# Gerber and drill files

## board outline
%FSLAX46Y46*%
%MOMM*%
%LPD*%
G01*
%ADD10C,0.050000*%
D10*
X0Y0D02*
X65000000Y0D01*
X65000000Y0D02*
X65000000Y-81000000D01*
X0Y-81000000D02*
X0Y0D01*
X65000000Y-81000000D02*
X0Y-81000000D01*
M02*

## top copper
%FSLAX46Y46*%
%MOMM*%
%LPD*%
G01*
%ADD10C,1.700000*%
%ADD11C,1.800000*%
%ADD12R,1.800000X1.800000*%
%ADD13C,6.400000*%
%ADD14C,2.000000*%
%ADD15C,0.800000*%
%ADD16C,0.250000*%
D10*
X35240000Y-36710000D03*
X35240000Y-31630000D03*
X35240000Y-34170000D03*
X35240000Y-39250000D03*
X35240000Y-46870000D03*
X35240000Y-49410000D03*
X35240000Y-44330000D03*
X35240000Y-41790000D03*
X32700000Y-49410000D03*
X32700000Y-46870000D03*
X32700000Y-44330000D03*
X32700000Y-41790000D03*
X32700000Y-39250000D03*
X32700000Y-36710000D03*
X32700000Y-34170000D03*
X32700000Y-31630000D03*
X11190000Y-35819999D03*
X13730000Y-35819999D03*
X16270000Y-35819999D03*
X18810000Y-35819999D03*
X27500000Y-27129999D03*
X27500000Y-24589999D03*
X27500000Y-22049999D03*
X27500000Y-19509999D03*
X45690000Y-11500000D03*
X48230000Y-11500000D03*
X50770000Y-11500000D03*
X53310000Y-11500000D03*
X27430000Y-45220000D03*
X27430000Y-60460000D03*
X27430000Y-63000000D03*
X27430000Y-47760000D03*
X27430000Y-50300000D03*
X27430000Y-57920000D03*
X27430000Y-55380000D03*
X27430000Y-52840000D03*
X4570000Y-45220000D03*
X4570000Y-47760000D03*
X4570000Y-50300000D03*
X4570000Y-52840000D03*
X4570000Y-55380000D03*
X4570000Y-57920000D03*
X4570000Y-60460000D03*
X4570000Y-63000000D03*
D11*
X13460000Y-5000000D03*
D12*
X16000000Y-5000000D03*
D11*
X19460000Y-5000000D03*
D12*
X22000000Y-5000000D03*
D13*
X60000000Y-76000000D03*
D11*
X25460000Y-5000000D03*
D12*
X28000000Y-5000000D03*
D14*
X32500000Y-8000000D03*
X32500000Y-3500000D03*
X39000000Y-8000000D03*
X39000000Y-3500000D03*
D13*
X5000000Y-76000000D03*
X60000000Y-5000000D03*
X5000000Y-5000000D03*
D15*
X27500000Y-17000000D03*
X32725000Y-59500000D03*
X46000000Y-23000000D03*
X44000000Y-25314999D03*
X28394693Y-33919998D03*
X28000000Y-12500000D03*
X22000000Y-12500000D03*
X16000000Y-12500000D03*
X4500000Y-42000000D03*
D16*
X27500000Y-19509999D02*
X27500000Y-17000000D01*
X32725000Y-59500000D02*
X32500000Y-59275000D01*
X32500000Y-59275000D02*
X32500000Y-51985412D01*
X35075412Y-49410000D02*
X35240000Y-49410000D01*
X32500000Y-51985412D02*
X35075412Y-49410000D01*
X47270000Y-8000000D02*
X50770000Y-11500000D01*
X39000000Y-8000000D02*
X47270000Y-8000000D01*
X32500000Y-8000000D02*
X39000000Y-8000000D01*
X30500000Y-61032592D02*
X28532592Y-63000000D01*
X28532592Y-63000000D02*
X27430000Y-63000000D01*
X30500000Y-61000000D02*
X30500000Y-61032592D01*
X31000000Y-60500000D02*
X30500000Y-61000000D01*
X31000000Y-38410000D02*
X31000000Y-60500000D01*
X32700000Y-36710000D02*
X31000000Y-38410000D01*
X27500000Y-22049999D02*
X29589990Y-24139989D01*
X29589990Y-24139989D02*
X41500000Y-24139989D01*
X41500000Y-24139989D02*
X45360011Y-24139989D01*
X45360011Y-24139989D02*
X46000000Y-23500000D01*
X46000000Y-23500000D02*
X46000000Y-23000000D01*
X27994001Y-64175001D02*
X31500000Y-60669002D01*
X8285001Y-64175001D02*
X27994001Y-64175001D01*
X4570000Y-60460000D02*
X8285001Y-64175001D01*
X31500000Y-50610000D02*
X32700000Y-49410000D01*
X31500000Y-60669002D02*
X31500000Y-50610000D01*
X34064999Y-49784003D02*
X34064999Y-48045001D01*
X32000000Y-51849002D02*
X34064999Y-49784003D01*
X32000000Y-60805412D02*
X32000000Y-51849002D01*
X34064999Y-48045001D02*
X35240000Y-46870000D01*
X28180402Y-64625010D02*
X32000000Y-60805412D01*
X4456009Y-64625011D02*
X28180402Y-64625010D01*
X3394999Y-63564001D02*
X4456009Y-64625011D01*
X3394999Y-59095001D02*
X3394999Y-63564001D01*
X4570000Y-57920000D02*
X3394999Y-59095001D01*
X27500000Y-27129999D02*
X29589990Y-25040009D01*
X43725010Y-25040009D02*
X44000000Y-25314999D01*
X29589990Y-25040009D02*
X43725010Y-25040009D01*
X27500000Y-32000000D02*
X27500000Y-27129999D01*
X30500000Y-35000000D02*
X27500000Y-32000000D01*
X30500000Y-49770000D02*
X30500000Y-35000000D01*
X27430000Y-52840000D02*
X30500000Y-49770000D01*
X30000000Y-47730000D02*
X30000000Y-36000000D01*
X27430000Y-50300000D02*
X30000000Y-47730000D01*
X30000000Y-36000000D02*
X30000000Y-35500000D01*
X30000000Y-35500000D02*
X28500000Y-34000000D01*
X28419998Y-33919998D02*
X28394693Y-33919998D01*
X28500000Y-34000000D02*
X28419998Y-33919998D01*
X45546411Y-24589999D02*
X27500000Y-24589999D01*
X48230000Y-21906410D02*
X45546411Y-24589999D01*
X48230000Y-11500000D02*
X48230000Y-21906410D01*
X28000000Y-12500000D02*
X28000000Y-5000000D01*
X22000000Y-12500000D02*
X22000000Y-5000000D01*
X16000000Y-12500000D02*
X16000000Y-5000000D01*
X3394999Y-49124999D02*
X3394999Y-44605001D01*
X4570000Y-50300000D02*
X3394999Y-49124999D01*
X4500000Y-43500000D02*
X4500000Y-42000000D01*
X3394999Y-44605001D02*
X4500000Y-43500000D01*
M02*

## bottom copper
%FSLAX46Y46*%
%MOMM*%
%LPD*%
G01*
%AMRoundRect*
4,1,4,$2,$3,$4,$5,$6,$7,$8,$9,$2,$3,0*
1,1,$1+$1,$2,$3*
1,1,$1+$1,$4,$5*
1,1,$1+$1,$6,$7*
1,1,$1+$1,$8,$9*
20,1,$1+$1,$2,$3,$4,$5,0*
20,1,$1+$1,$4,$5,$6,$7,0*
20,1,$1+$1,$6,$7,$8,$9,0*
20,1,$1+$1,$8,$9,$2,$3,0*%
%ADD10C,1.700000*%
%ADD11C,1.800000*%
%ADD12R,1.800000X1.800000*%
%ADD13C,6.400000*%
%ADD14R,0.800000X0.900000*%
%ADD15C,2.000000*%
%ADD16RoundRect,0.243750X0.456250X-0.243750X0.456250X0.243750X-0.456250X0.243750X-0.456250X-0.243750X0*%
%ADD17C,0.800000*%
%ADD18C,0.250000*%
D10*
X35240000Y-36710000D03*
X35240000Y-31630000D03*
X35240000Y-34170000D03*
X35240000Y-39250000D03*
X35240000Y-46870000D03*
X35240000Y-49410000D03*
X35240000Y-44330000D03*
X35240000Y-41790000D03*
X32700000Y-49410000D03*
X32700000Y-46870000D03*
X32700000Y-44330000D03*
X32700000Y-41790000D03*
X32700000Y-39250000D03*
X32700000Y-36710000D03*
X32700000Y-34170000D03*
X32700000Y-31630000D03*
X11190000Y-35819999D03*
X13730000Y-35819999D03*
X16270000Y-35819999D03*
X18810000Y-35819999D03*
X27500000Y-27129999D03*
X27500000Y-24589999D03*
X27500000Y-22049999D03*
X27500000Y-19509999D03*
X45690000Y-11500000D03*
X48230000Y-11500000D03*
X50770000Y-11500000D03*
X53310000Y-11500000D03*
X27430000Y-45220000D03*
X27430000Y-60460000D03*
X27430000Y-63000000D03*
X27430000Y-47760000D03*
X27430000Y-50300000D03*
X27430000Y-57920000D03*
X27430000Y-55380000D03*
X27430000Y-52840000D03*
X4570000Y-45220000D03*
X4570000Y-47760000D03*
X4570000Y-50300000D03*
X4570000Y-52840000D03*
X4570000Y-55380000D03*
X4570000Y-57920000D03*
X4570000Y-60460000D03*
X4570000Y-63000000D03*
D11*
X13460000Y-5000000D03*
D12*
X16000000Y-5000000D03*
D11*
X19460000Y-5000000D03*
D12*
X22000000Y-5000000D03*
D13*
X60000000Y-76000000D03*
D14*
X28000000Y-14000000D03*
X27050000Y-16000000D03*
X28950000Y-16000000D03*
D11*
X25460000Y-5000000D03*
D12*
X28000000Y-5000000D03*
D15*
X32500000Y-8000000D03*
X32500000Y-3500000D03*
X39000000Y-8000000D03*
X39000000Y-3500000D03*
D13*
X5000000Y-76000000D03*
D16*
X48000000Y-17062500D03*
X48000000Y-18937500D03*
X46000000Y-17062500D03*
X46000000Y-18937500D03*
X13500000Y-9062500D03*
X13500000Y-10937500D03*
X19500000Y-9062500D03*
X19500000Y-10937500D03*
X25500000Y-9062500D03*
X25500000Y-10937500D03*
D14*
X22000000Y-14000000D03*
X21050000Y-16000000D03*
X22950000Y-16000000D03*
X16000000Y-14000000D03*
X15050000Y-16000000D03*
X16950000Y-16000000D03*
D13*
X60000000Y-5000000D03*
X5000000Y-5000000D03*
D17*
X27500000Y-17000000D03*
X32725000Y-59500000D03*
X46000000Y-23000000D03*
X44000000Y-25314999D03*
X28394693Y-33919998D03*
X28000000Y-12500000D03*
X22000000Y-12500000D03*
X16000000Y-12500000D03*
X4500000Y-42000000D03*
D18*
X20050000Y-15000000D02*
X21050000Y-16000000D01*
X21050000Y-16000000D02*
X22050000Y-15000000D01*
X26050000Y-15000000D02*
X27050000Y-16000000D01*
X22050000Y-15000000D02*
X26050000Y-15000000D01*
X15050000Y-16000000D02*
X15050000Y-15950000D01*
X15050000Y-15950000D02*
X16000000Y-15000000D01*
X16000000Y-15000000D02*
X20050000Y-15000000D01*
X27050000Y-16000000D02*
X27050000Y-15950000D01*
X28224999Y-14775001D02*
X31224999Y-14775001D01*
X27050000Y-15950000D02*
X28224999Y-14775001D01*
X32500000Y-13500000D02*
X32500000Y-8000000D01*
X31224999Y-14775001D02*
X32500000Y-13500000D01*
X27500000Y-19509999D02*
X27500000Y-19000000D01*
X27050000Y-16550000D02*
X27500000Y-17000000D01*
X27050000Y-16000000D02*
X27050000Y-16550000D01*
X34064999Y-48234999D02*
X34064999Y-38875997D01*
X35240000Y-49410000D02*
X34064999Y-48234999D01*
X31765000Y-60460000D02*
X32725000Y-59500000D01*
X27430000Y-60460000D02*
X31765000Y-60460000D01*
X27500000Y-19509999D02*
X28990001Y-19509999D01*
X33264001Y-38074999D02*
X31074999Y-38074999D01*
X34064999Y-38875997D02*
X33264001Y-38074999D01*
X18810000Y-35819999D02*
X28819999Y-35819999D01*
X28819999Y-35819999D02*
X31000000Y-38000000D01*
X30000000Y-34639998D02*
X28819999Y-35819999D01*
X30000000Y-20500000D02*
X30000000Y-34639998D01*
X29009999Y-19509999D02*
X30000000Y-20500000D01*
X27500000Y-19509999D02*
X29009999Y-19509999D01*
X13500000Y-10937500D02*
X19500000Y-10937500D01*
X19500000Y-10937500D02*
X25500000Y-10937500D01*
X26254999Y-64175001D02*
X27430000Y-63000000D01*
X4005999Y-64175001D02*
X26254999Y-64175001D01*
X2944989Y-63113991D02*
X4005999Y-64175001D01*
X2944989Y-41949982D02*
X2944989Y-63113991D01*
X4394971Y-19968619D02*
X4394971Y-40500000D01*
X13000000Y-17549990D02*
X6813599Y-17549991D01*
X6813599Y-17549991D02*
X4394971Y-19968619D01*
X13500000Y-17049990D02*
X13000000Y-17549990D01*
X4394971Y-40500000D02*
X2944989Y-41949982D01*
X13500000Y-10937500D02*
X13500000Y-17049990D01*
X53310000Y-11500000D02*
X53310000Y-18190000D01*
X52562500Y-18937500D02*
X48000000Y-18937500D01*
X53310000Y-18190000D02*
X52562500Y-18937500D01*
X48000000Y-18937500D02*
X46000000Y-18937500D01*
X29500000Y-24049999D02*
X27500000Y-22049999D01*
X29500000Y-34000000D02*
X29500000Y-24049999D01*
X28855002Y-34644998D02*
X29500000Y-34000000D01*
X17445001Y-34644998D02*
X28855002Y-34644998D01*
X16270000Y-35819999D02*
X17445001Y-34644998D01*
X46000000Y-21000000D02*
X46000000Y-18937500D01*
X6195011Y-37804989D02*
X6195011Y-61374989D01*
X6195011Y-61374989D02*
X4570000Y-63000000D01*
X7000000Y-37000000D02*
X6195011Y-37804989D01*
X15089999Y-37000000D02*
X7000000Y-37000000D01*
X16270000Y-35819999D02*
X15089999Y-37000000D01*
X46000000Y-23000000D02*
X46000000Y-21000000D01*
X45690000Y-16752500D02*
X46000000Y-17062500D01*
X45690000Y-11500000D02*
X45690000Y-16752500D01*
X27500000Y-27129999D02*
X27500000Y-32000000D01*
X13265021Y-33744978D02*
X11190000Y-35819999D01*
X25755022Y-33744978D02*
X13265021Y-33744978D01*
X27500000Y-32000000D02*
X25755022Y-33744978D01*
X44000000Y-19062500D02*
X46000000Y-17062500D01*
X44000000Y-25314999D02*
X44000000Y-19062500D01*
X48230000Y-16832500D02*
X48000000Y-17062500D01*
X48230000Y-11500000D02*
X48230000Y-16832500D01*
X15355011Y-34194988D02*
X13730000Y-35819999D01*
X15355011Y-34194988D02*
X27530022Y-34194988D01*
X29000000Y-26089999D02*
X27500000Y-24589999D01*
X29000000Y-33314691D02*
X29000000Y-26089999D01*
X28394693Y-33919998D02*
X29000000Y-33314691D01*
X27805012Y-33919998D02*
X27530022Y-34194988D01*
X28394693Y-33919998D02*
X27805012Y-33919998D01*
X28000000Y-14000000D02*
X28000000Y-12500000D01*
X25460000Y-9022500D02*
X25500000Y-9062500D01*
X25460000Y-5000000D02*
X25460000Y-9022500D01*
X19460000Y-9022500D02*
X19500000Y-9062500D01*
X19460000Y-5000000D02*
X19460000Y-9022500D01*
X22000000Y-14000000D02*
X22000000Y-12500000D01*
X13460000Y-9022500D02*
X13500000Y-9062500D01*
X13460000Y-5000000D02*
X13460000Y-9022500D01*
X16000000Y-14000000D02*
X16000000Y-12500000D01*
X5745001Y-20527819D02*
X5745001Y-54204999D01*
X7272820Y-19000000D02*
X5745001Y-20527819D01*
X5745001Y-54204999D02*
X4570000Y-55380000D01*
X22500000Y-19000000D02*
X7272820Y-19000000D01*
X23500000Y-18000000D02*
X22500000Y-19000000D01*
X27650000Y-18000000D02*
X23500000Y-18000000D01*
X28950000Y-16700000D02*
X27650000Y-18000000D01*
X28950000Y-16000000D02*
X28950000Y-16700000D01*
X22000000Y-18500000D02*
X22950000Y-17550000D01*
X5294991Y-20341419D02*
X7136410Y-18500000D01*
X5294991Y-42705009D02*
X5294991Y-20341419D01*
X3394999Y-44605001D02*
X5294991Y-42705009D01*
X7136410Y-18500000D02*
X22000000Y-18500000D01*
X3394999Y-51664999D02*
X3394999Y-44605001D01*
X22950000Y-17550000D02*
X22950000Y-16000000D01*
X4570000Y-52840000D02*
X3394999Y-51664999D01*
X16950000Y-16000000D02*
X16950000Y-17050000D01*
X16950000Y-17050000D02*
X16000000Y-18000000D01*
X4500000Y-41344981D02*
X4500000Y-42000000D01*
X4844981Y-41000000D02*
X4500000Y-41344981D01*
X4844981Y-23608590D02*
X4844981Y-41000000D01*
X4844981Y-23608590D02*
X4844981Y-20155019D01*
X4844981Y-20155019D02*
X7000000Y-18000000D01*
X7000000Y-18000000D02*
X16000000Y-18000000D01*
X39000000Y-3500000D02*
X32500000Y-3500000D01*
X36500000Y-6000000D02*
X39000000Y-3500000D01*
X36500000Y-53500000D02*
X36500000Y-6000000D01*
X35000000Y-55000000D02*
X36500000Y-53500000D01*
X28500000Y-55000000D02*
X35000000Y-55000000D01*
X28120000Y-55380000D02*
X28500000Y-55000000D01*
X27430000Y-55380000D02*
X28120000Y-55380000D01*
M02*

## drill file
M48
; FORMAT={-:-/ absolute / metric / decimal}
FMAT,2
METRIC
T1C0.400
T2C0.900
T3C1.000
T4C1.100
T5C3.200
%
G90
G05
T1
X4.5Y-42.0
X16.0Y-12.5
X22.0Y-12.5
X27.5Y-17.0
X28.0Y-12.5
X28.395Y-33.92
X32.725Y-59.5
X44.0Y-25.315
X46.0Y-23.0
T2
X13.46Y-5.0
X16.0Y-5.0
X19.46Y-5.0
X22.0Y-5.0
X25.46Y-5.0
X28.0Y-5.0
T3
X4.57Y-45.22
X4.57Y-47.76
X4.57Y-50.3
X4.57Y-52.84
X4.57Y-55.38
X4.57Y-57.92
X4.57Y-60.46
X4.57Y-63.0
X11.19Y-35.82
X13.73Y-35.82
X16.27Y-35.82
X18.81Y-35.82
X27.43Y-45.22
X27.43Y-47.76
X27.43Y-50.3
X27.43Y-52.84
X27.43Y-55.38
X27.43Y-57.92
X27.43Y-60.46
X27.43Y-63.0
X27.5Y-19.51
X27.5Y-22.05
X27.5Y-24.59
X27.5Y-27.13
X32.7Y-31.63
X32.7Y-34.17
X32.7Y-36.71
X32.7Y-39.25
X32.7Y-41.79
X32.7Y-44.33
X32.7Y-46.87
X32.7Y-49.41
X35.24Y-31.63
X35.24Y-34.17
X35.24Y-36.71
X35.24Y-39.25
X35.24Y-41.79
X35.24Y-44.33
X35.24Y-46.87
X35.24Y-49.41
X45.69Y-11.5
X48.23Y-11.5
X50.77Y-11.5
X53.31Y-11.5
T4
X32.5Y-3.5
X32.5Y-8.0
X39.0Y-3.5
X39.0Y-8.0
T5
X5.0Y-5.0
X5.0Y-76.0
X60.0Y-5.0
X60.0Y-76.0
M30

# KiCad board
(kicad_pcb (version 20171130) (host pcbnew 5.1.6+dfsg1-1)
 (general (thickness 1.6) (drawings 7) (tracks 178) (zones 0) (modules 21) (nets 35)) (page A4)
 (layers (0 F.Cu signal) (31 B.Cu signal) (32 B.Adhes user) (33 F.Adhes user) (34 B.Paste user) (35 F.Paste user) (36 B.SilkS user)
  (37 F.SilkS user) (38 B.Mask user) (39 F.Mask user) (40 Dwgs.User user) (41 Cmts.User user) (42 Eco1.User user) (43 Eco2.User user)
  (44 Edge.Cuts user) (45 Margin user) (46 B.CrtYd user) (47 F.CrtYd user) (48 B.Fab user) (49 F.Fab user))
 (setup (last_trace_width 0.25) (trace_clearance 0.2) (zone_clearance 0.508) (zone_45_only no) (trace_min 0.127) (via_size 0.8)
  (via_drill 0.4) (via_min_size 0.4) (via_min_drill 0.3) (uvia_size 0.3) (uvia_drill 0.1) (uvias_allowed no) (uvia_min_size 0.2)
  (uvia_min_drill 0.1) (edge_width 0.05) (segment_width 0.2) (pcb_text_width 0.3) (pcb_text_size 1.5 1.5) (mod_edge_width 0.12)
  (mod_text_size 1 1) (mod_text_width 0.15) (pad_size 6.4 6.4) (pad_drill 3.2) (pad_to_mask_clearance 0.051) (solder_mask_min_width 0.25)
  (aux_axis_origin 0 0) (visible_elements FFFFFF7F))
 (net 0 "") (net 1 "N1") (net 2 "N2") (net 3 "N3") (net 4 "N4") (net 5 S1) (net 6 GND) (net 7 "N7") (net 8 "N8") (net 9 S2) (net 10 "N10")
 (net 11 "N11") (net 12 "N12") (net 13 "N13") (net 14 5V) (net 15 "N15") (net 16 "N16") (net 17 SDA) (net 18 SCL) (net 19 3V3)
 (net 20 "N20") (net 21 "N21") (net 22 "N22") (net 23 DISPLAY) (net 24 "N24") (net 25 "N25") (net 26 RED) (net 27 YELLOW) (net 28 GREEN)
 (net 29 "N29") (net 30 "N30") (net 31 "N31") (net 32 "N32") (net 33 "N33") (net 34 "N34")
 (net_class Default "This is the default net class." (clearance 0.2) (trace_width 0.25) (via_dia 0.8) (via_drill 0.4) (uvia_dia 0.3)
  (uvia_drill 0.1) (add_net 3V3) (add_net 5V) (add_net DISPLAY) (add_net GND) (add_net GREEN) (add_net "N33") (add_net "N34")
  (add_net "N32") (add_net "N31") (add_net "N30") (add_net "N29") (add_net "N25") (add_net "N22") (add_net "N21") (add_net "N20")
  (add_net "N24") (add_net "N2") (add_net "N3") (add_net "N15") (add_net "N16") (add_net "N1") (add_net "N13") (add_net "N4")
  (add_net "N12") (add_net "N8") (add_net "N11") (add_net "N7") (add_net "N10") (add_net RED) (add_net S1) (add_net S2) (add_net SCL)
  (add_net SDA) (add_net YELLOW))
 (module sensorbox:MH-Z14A (layer F.Cu) (at 65 14.5 270)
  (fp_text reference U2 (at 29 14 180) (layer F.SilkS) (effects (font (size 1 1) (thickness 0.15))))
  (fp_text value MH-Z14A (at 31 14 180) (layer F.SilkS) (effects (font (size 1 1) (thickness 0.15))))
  (pad 2 thru_hole circle (at 22.21 29.76 270) (size 1.7 1.7) (drill 1) (layers *.Cu *.Mask) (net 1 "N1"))
  (pad 14 thru_hole circle (at 17.13 29.76 270) (size 1.7 1.7) (drill 1) (layers *.Cu *.Mask) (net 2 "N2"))
  (pad 15 thru_hole circle (at 19.67 29.76 270) (size 1.7 1.7) (drill 1) (layers *.Cu *.Mask) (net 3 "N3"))
  (pad 4 thru_hole circle (at 24.75 29.76 270) (size 1.7 1.7) (drill 1) (layers *.Cu *.Mask) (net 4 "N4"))
  (pad 10 thru_hole circle (at 32.37 29.76 270) (size 1.7 1.7) (drill 1) (layers *.Cu *.Mask) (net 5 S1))
  (pad 12 thru_hole circle (at 34.91 29.76 270) (size 1.7 1.7) (drill 1) (layers *.Cu *.Mask) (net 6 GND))
  (pad 8 thru_hole circle (at 29.83 29.76 270) (size 1.7 1.7) (drill 1) (layers *.Cu *.Mask) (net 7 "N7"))
  (pad 6 thru_hole circle (at 27.29 29.76 270) (size 1.7 1.7) (drill 1) (layers *.Cu *.Mask) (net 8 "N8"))
  (pad 11 thru_hole circle (at 34.91 32.3 270) (size 1.7 1.7) (drill 1) (layers *.Cu *.Mask) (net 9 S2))
  (pad 9 thru_hole circle (at 32.37 32.3 270) (size 1.7 1.7) (drill 1) (layers *.Cu *.Mask) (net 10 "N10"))
  (pad 7 thru_hole circle (at 29.83 32.3 270) (size 1.7 1.7) (drill 1) (layers *.Cu *.Mask) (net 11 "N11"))
  (pad 5 thru_hole circle (at 27.29 32.3 270) (size 1.7 1.7) (drill 1) (layers *.Cu *.Mask) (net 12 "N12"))
  (pad 3 thru_hole circle (at 24.75 32.3 270) (size 1.7 1.7) (drill 1) (layers *.Cu *.Mask) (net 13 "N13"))
  (pad 1 thru_hole circle (at 22.21 32.3 270) (size 1.7 1.7) (drill 1) (layers *.Cu *.Mask) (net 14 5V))
  (pad 16 thru_hole circle (at 19.67 32.3 270) (size 1.7 1.7) (drill 1) (layers *.Cu *.Mask) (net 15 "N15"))
  (pad 17 thru_hole circle (at 17.13 32.3 270) (size 1.7 1.7) (drill 1) (layers *.Cu *.Mask) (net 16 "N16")))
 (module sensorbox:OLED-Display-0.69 (layer F.Cu) (at 15 23.319999 180)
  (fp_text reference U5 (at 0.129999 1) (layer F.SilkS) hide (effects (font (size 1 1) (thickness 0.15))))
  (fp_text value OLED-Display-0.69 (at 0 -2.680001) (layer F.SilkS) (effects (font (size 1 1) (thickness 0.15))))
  (pad 4 thru_hole circle (at 3.81 -12.5 180) (size 1.7 1.7) (drill 1) (layers *.Cu *.Mask) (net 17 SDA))
  (pad 3 thru_hole circle (at 1.27 -12.5 180) (size 1.7 1.7) (drill 1) (layers *.Cu *.Mask) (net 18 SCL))
  (pad 2 thru_hole circle (at -1.27 -12.5 180) (size 1.7 1.7) (drill 1) (layers *.Cu *.Mask) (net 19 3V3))
  (pad 1 thru_hole circle (at -3.81 -12.5 180) (size 1.7 1.7) (drill 1) (layers *.Cu *.Mask) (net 6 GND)))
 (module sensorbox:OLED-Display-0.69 (layer F.Cu) (at 15 23.319999 270)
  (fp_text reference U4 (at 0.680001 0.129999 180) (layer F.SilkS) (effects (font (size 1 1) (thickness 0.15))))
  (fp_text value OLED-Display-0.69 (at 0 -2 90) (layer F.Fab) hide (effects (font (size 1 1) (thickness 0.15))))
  (pad 4 thru_hole circle (at 3.81 -12.5 270) (size 1.7 1.7) (drill 1) (layers *.Cu *.Mask) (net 17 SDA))
  (pad 3 thru_hole circle (at 1.27 -12.5 270) (size 1.7 1.7) (drill 1) (layers *.Cu *.Mask) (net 18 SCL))
  (pad 2 thru_hole circle (at -1.27 -12.5 270) (size 1.7 1.7) (drill 1) (layers *.Cu *.Mask) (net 19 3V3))
  (pad 1 thru_hole circle (at -3.81 -12.5 270) (size 1.7 1.7) (drill 1) (layers *.Cu *.Mask) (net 6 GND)))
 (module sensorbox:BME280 (layer F.Cu) (at 49.5 7 180)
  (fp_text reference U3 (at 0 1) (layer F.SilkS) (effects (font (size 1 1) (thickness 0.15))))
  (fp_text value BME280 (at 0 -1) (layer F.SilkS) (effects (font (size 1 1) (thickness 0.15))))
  (pad 4 thru_hole circle (at 3.81 -4.5 180) (size 1.7 1.7) (drill 1) (layers *.Cu *.Mask) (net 17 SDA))
  (pad 3 thru_hole circle (at 1.27 -4.5 180) (size 1.7 1.7) (drill 1) (layers *.Cu *.Mask) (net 18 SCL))
  (pad 2 thru_hole circle (at -1.27 -4.5 180) (size 1.7 1.7) (drill 1) (layers *.Cu *.Mask) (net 6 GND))
  (pad 1 thru_hole circle (at -3.81 -4.5 180) (size 1.7 1.7) (drill 1) (layers *.Cu *.Mask) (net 19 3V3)))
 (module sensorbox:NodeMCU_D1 (layer F.Cu) (at 16 72 90)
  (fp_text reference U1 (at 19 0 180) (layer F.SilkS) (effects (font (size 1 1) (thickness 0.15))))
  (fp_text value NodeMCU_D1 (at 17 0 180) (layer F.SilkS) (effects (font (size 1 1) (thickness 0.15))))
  (pad 8 thru_hole circle (at 26.78 11.43 90) (size 1.7 1.7) (drill 1) (layers *.Cu *.Mask) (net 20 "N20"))
  (pad 2 thru_hole circle (at 11.54 11.43 90) (size 1.7 1.7) (drill 1) (layers *.Cu *.Mask) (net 6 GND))
  (pad 1 thru_hole circle (at 9 11.43 90) (size 1.7 1.7) (drill 1) (layers *.Cu *.Mask) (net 14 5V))
  (pad 7 thru_hole circle (at 24.24 11.43 90) (size 1.7 1.7) (drill 1) (layers *.Cu *.Mask) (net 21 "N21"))
  (pad 6 thru_hole circle (at 21.7 11.43 90) (size 1.7 1.7) (drill 1) (layers *.Cu *.Mask) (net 18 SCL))
  (pad 3 thru_hole circle (at 14.08 11.43 90) (size 1.7 1.7) (drill 1) (layers *.Cu *.Mask) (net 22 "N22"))
  (pad 4 thru_hole circle (at 16.62 11.43 90) (size 1.7 1.7) (drill 1) (layers *.Cu *.Mask) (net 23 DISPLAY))
  (pad 5 thru_hole circle (at 19.16 11.43 90) (size 1.7 1.7) (drill 1) (layers *.Cu *.Mask) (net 17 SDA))
  (pad 9 thru_hole circle (at 26.78 -11.43 90) (size 1.7 1.7) (drill 1) (layers *.Cu *.Mask) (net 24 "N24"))
  (pad 10 thru_hole circle (at 24.24 -11.43 90) (size 1.7 1.7) (drill 1) (layers *.Cu *.Mask) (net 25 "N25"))
  (pad 11 thru_hole circle (at 21.7 -11.43 90) (size 1.7 1.7) (drill 1) (layers *.Cu *.Mask) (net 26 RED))
  (pad 12 thru_hole circle (at 19.16 -11.43 90) (size 1.7 1.7) (drill 1) (layers *.Cu *.Mask) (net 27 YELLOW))
  (pad 13 thru_hole circle (at 16.62 -11.43 90) (size 1.7 1.7) (drill 1) (layers *.Cu *.Mask) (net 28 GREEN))
  (pad 14 thru_hole circle (at 14.08 -11.43 90) (size 1.7 1.7) (drill 1) (layers *.Cu *.Mask) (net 5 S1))
  (pad 15 thru_hole circle (at 11.54 -11.43 90) (size 1.7 1.7) (drill 1) (layers *.Cu *.Mask) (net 9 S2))
  (pad 16 thru_hole circle (at 9 -11.43 90) (size 1.7 1.7) (drill 1) (layers *.Cu *.Mask) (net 19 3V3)))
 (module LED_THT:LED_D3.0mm (layer F.Cu) (at 16 5 180)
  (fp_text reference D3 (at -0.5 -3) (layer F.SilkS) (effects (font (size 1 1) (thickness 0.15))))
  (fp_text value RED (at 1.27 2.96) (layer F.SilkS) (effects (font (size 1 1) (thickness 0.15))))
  (pad 2 thru_hole circle (at 2.54 0 180) (size 1.8 1.8) (drill 0.9) (layers *.Cu *.Mask) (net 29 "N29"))
  (pad 1 thru_hole rect (at 0 0 180) (size 1.8 1.8) (drill 0.9) (layers *.Cu *.Mask) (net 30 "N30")))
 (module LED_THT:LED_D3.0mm (layer F.Cu) (at 22 5 180)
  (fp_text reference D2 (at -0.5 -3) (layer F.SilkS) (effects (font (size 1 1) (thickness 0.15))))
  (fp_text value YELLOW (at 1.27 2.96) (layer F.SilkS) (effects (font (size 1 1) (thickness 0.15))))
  (pad 2 thru_hole circle (at 2.54 0 180) (size 1.8 1.8) (drill 0.9) (layers *.Cu *.Mask) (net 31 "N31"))
  (pad 1 thru_hole rect (at 0 0 180) (size 1.8 1.8) (drill 0.9) (layers *.Cu *.Mask) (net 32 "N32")))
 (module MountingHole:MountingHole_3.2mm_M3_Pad (layer F.Cu) (at 60 76)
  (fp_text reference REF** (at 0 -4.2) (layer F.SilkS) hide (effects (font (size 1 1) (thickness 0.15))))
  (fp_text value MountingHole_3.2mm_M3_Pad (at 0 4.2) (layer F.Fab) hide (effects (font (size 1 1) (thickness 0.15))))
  (pad 1 thru_hole circle (at 0 0) (size 6.4 6.4) (drill 3.2) (layers *.Cu *.Mask)))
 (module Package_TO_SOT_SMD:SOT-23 (layer B.Cu) (at 28 15 90)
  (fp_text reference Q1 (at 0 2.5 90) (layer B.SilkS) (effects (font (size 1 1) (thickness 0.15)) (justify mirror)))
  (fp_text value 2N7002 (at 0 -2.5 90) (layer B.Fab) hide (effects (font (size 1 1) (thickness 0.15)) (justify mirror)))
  (pad 3 smd rect (at 1 0 90) (size 0.9 0.8) (layers B.Cu B.Paste B.Mask) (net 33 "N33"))
  (pad 2 smd rect (at -1 -0.95 90) (size 0.9 0.8) (layers B.Cu B.Paste B.Mask) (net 6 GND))
  (pad 1 smd rect (at -1 0.95 90) (size 0.9 0.8) (layers B.Cu B.Paste B.Mask) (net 28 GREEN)))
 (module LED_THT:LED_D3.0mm (layer F.Cu) (at 28 5 180)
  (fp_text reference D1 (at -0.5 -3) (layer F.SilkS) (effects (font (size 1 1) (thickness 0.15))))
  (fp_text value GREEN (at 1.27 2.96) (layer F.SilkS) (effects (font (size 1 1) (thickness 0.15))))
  (pad 2 thru_hole circle (at 2.54 0 180) (size 1.8 1.8) (drill 0.9) (layers *.Cu *.Mask) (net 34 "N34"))
  (pad 1 thru_hole rect (at 0 0 180) (size 1.8 1.8) (drill 0.9) (layers *.Cu *.Mask) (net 33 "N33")))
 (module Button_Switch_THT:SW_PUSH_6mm (layer F.Cu) (at 39 8 180)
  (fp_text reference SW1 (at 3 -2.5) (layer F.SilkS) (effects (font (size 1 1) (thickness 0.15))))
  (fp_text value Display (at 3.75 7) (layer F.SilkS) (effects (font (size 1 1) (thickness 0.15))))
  (pad 1 thru_hole circle (at 6.5 0 270) (size 2 2) (drill 1.1) (layers *.Cu *.Mask) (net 6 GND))
  (pad 2 thru_hole circle (at 6.5 4.5 270) (size 2 2) (drill 1.1) (layers *.Cu *.Mask) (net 23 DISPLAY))
  (pad 1 thru_hole circle (at 0 0 270) (size 2 2) (drill 1.1) (layers *.Cu *.Mask) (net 6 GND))
  (pad 2 thru_hole circle (at 0 4.5 270) (size 2 2) (drill 1.1) (layers *.Cu *.Mask) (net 23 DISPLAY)))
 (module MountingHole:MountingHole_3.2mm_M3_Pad (layer F.Cu) (at 5 76)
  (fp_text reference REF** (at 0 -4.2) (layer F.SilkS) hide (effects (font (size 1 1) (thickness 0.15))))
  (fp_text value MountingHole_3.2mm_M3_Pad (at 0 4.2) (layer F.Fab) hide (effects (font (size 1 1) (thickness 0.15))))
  (pad 1 thru_hole circle (at 0 0) (size 6.4 6.4) (drill 3.2) (layers *.Cu *.Mask)))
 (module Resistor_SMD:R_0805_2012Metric (layer B.Cu) (at 48 18 90)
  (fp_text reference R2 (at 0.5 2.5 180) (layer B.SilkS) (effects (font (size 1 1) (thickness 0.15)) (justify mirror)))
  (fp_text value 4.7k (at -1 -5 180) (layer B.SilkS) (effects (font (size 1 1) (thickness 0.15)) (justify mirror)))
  (pad 2 smd roundrect (at 0.9375 0 90) (size 0.975 1.4) (layers B.Cu B.Paste B.Mask) (roundrect_rratio 0.25) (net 18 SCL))
  (pad 1 smd roundrect (at -0.9375 0 90) (size 0.975 1.4) (layers B.Cu B.Paste B.Mask) (roundrect_rratio 0.25) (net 19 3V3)))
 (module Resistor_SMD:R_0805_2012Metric (layer B.Cu) (at 46 18 90)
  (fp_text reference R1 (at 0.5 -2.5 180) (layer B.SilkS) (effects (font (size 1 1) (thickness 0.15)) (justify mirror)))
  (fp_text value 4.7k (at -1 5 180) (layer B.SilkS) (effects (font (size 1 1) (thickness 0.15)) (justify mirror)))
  (pad 2 smd roundrect (at 0.9375 0 90) (size 0.975 1.4) (layers B.Cu B.Paste B.Mask) (roundrect_rratio 0.25) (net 17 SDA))
  (pad 1 smd roundrect (at -0.9375 0 90) (size 0.975 1.4) (layers B.Cu B.Paste B.Mask) (roundrect_rratio 0.25) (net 19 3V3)))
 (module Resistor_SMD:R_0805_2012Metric (layer B.Cu) (at 13.5 10 90)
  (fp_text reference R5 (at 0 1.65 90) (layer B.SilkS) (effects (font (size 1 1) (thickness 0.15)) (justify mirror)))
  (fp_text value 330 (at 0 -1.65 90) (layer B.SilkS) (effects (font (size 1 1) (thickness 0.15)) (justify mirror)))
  (pad 2 smd roundrect (at 0.9375 0 90) (size 0.975 1.4) (layers B.Cu B.Paste B.Mask) (roundrect_rratio 0.25) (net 29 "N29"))
  (pad 1 smd roundrect (at -0.9375 0 90) (size 0.975 1.4) (layers B.Cu B.Paste B.Mask) (roundrect_rratio 0.25) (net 14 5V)))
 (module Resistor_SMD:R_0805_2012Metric (layer B.Cu) (at 19.5 10 90)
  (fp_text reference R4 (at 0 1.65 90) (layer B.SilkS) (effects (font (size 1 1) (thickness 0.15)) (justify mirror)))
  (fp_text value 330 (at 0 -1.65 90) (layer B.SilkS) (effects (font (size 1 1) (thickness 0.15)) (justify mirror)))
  (pad 2 smd roundrect (at 0.9375 0 90) (size 0.975 1.4) (layers B.Cu B.Paste B.Mask) (roundrect_rratio 0.25) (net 31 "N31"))
  (pad 1 smd roundrect (at -0.9375 0 90) (size 0.975 1.4) (layers B.Cu B.Paste B.Mask) (roundrect_rratio 0.25) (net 14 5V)))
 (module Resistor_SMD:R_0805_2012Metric (layer B.Cu) (at 25.5 10 90)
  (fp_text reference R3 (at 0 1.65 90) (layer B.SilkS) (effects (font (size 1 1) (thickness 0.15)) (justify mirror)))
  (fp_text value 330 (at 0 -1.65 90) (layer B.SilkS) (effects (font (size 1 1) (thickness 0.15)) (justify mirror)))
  (pad 2 smd roundrect (at 0.9375 0 90) (size 0.975 1.4) (layers B.Cu B.Paste B.Mask) (roundrect_rratio 0.25) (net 34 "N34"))
  (pad 1 smd roundrect (at -0.9375 0 90) (size 0.975 1.4) (layers B.Cu B.Paste B.Mask) (roundrect_rratio 0.25) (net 14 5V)))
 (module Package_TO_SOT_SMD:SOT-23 (layer B.Cu) (at 22 15 90)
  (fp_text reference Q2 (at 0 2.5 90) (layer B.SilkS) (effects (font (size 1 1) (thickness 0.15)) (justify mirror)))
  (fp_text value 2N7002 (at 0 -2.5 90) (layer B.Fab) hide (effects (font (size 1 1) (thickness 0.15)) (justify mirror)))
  (pad 3 smd rect (at 1 0 90) (size 0.9 0.8) (layers B.Cu B.Paste B.Mask) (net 32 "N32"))
  (pad 2 smd rect (at -1 -0.95 90) (size 0.9 0.8) (layers B.Cu B.Paste B.Mask) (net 6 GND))
  (pad 1 smd rect (at -1 0.95 90) (size 0.9 0.8) (layers B.Cu B.Paste B.Mask) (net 27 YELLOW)))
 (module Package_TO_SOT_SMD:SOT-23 (layer B.Cu) (at 16 15 90)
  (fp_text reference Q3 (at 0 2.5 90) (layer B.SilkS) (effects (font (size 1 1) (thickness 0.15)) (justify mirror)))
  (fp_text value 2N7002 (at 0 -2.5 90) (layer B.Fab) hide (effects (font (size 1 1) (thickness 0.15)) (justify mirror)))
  (pad 3 smd rect (at 1 0 90) (size 0.9 0.8) (layers B.Cu B.Paste B.Mask) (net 30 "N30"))
  (pad 2 smd rect (at -1 -0.95 90) (size 0.9 0.8) (layers B.Cu B.Paste B.Mask) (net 6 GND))
  (pad 1 smd rect (at -1 0.95 90) (size 0.9 0.8) (layers B.Cu B.Paste B.Mask) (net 26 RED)))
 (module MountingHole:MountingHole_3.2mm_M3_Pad (layer F.Cu) (at 60 5)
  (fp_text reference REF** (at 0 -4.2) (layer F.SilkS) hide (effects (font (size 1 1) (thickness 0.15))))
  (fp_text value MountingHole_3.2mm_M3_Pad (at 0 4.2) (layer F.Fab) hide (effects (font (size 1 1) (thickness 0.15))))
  (pad 1 thru_hole circle (at 0 0) (size 6.4 6.4) (drill 3.2) (layers *.Cu *.Mask)))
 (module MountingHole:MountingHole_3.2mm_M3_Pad (layer F.Cu) (at 5 5)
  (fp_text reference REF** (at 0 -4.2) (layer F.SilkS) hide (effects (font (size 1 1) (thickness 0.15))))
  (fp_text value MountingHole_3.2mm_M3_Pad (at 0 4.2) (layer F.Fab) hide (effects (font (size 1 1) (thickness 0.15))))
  (pad 1 thru_hole circle (at 0 0) (size 6.4 6.4) (drill 3.2) (layers *.Cu *.Mask)))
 (gr_line (start 0 0) (end 65 0) (layer Edge.Cuts) (width 0.05))
 (gr_line (start 65 0) (end 65 81) (layer Edge.Cuts) (width 0.05))
 (gr_line (start 0 81) (end 0 0) (layer Edge.Cuts) (width 0.05))
 (gr_line (start 65 81) (end 0 81) (layer Edge.Cuts) (width 0.05))
 (segment (start 20.05 15) (end 21.05 16) (width 0.25) (layer B.Cu) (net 6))
 (segment (start 21.05 16) (end 22.05 15) (width 0.25) (layer B.Cu) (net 6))
 (segment (start 26.05 15) (end 27.05 16) (width 0.25) (layer B.Cu) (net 6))
 (segment (start 22.05 15) (end 26.05 15) (width 0.25) (layer B.Cu) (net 6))
 (segment (start 15.05 16) (end 15.05 15.95) (width 0.25) (layer B.Cu) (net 6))
 (segment (start 15.05 15.95) (end 16 15) (width 0.25) (layer B.Cu) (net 6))
 (segment (start 16 15) (end 20.05 15) (width 0.25) (layer B.Cu) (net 6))
 (segment (start 27.05 16) (end 27.05 15.95) (width 0.25) (layer B.Cu) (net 6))
 (segment (start 28.224999 14.775001) (end 31.224999 14.775001) (width 0.25) (layer B.Cu) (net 6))
 (segment (start 27.05 15.95) (end 28.224999 14.775001) (width 0.25) (layer B.Cu) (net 6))
 (segment (start 32.5 13.5) (end 32.5 8) (width 0.25) (layer B.Cu) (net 6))
 (segment (start 31.224999 14.775001) (end 32.5 13.5) (width 0.25) (layer B.Cu) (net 6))
 (segment (start 27.5 19.509999) (end 27.5 19) (width 0.25) (layer B.Cu) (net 6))
 (via (at 27.5 17) (size 0.8) (drill 0.4) (layers F.Cu B.Cu) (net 6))
 (segment (start 27.5 19.509999) (end 27.5 17) (width 0.25) (layer F.Cu) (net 6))
 (segment (start 27.05 16.55) (end 27.5 17) (width 0.25) (layer B.Cu) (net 6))
 (segment (start 27.05 16) (end 27.05 16.55) (width 0.25) (layer B.Cu) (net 6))
 (segment (start 34.064999 48.234999) (end 34.064999 38.875997) (width 0.25) (layer B.Cu) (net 6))
 (segment (start 35.24 49.41) (end 34.064999 48.234999) (width 0.25) (layer B.Cu) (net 6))
 (via (at 32.725 59.5) (size 0.8) (drill 0.4) (layers F.Cu B.Cu) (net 6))
 (segment (start 31.765 60.46) (end 32.725 59.5) (width 0.25) (layer B.Cu) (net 6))
 (segment (start 27.43 60.46) (end 31.765 60.46) (width 0.25) (layer B.Cu) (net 6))
 (segment (start 32.725 59.5) (end 32.5 59.275) (width 0.25) (layer F.Cu) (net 6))
 (segment (start 32.5 59.275) (end 32.5 51.985412) (width 0.25) (layer F.Cu) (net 6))
 (segment (start 35.075412 49.41) (end 35.24 49.41) (width 0.25) (layer F.Cu) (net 6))
 (segment (start 32.5 51.985412) (end 35.075412 49.41) (width 0.25) (layer F.Cu) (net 6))
 (segment (start 47.27 8) (end 50.77 11.5) (width 0.25) (layer F.Cu) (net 6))
 (segment (start 39 8) (end 47.27 8) (width 0.25) (layer F.Cu) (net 6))
 (segment (start 32.5 8) (end 39 8) (width 0.25) (layer F.Cu) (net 6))
 (segment (start 27.5 19.509999) (end 28.990001 19.509999) (width 0.25) (layer B.Cu) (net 6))
 (segment (start 33.264001 38.074999) (end 31.074999 38.074999) (width 0.25) (layer B.Cu) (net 6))
 (segment (start 34.064999 38.875997) (end 33.264001 38.074999) (width 0.25) (layer B.Cu) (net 6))
 (segment (start 18.81 35.819999) (end 28.819999 35.819999) (width 0.25) (layer B.Cu) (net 6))
 (segment (start 28.819999 35.819999) (end 31 38) (width 0.25) (layer B.Cu) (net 6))
 (segment (start 30 34.639998) (end 28.819999 35.819999) (width 0.25) (layer B.Cu) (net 6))
 (segment (start 30 20.5) (end 30 34.639998) (width 0.25) (layer B.Cu) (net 6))
 (segment (start 29.009999 19.509999) (end 30 20.5) (width 0.25) (layer B.Cu) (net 6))
 (segment (start 27.5 19.509999) (end 29.009999 19.509999) (width 0.25) (layer B.Cu) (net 6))
 (segment (start 13.5 10.9375) (end 19.5 10.9375) (width 0.25) (layer B.Cu) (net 14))
 (segment (start 19.5 10.9375) (end 25.5 10.9375) (width 0.25) (layer B.Cu) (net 14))
 (segment (start 26.254999 64.175001) (end 27.43 63) (width 0.25) (layer B.Cu) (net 14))
 (segment (start 4.005999 64.175001) (end 26.254999 64.175001) (width 0.25) (layer B.Cu) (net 14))
 (segment (start 2.944989 63.113991) (end 4.005999 64.175001) (width 0.25) (layer B.Cu) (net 14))
 (segment (start 2.944989 41.949982) (end 2.944989 63.113991) (width 0.25) (layer B.Cu) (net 14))
 (segment (start 4.394971 19.968619) (end 4.394971 40.5) (width 0.25) (layer B.Cu) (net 14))
 (segment (start 13 17.54999) (end 6.813599 17.549991) (width 0.25) (layer B.Cu) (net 14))
 (segment (start 6.813599 17.549991) (end 4.394971 19.968619) (width 0.25) (layer B.Cu) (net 14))
 (segment (start 13.5 17.04999) (end 13 17.54999) (width 0.25) (layer B.Cu) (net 14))
 (segment (start 4.394971 40.5) (end 2.944989 41.949982) (width 0.25) (layer B.Cu) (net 14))
 (segment (start 13.5 10.9375) (end 13.5 17.04999) (width 0.25) (layer B.Cu) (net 14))
 (segment (start 30.5 61.032592) (end 28.532592 63) (width 0.25) (layer F.Cu) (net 14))
 (segment (start 28.532592 63) (end 27.43 63) (width 0.25) (layer F.Cu) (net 14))
 (segment (start 30.5 61) (end 30.5 61.032592) (width 0.25) (layer F.Cu) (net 14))
 (segment (start 31 60.5) (end 30.5 61) (width 0.25) (layer F.Cu) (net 14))
 (segment (start 31 38.41) (end 31 60.5) (width 0.25) (layer F.Cu) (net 14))
 (segment (start 32.7 36.71) (end 31 38.41) (width 0.25) (layer F.Cu) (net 14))
 (segment (start 53.31 11.5) (end 53.31 18.19) (width 0.25) (layer B.Cu) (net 19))
 (segment (start 52.5625 18.9375) (end 48 18.9375) (width 0.25) (layer B.Cu) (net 19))
 (segment (start 53.31 18.19) (end 52.5625 18.9375) (width 0.25) (layer B.Cu) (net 19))
 (segment (start 48 18.9375) (end 46 18.9375) (width 0.25) (layer B.Cu) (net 19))
 (segment (start 29.5 24.049999) (end 27.5 22.049999) (width 0.25) (layer B.Cu) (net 19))
 (segment (start 29.5 34) (end 29.5 24.049999) (width 0.25) (layer B.Cu) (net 19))
 (segment (start 28.855002 34.644998) (end 29.5 34) (width 0.25) (layer B.Cu) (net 19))
 (segment (start 17.445001 34.644998) (end 28.855002 34.644998) (width 0.25) (layer B.Cu) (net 19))
 (segment (start 16.27 35.819999) (end 17.445001 34.644998) (width 0.25) (layer B.Cu) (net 19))
 (segment (start 46 21) (end 46 18.9375) (width 0.25) (layer B.Cu) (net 19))
 (segment (start 6.195011 37.804989) (end 6.195011 61.374989) (width 0.25) (layer B.Cu) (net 19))
 (segment (start 6.195011 61.374989) (end 4.57 63) (width 0.25) (layer B.Cu) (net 19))
 (segment (start 7 37) (end 6.195011 37.804989) (width 0.25) (layer B.Cu) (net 19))
 (segment (start 15.089999 37) (end 7 37) (width 0.25) (layer B.Cu) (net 19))
 (segment (start 16.27 35.819999) (end 15.089999 37) (width 0.25) (layer B.Cu) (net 19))
 (segment (start 27.5 22.049999) (end 29.58999 24.139989) (width 0.25) (layer F.Cu) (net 19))
 (segment (start 29.58999 24.139989) (end 41.5 24.139989) (width 0.25) (layer F.Cu) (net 19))
 (segment (start 41.5 24.139989) (end 45.360011 24.139989) (width 0.25) (layer F.Cu) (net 19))
 (segment (start 45.360011 24.139989) (end 46 23.5) (width 0.25) (layer F.Cu) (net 19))
 (via (at 46 23) (size 0.8) (drill 0.4) (layers F.Cu B.Cu) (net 19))
 (segment (start 46 23.5) (end 46 23) (width 0.25) (layer F.Cu) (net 19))
 (segment (start 46 23) (end 46 21) (width 0.25) (layer B.Cu) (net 19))
 (segment (start 27.994001 64.175001) (end 31.5 60.669002) (width 0.25) (layer F.Cu) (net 9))
 (segment (start 8.285001 64.175001) (end 27.994001 64.175001) (width 0.25) (layer F.Cu) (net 9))
 (segment (start 4.57 60.46) (end 8.285001 64.175001) (width 0.25) (layer F.Cu) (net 9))
 (segment (start 31.5 50.61) (end 32.7 49.41) (width 0.25) (layer F.Cu) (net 9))
 (segment (start 31.5 60.669002) (end 31.5 50.61) (width 0.25) (layer F.Cu) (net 9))
 (segment (start 34.064999 49.784003) (end 34.064999 48.045001) (width 0.25) (layer F.Cu) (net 5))
 (segment (start 32 51.849002) (end 34.064999 49.784003) (width 0.25) (layer F.Cu) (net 5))
 (segment (start 32 60.805412) (end 32 51.849002) (width 0.25) (layer F.Cu) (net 5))
 (segment (start 34.064999 48.045001) (end 35.24 46.87) (width 0.25) (layer F.Cu) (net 5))
 (segment (start 28.180402 64.62501) (end 32 60.805412) (width 0.25) (layer F.Cu) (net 5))
 (segment (start 4.456009 64.625011) (end 28.180402 64.62501) (width 0.25) (layer F.Cu) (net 5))
 (segment (start 3.394999 63.564001) (end 4.456009 64.625011) (width 0.25) (layer F.Cu) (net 5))
 (segment (start 3.394999 59.095001) (end 3.394999 63.564001) (width 0.25) (layer F.Cu) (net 5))
 (segment (start 4.57 57.92) (end 3.394999 59.095001) (width 0.25) (layer F.Cu) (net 5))
 (segment (start 45.69 16.7525) (end 46 17.0625) (width 0.25) (layer B.Cu) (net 17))
 (segment (start 45.69 11.5) (end 45.69 16.7525) (width 0.25) (layer B.Cu) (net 17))
 (segment (start 27.5 27.129999) (end 27.5 32) (width 0.25) (layer B.Cu) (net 17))
 (segment (start 13.265021 33.744978) (end 11.19 35.819999) (width 0.25) (layer B.Cu) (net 17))
 (segment (start 25.755022 33.744978) (end 13.265021 33.744978) (width 0.25) (layer B.Cu) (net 17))
 (segment (start 27.5 32) (end 25.755022 33.744978) (width 0.25) (layer B.Cu) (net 17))
 (segment (start 27.5 27.129999) (end 29.58999 25.040009) (width 0.25) (layer F.Cu) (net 17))
 (via (at 44 25.314999) (size 0.8) (drill 0.4) (layers F.Cu B.Cu) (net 17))
 (segment (start 43.72501 25.040009) (end 44 25.314999) (width 0.25) (layer F.Cu) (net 17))
 (segment (start 29.58999 25.040009) (end 43.72501 25.040009) (width 0.25) (layer F.Cu) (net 17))
 (segment (start 44 19.0625) (end 46 17.0625) (width 0.25) (layer B.Cu) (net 17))
 (segment (start 44 25.314999) (end 44 19.0625) (width 0.25) (layer B.Cu) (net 17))
 (segment (start 27.5 32) (end 27.5 27.129999) (width 0.25) (layer F.Cu) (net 17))
 (segment (start 30.5 35) (end 27.5 32) (width 0.25) (layer F.Cu) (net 17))
 (segment (start 30.5 49.77) (end 30.5 35) (width 0.25) (layer F.Cu) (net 17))
 (segment (start 27.43 52.84) (end 30.5 49.77) (width 0.25) (layer F.Cu) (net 17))
 (segment (start 48.23 16.8325) (end 48 17.0625) (width 0.25) (layer B.Cu) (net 18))
 (segment (start 48.23 11.5) (end 48.23 16.8325) (width 0.25) (layer B.Cu) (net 18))
 (segment (start 15.355011 34.194988) (end 13.73 35.819999) (width 0.25) (layer B.Cu) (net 18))
 (segment (start 30 47.73) (end 30 36) (width 0.25) (layer F.Cu) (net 18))
 (segment (start 27.43 50.3) (end 30 47.73) (width 0.25) (layer F.Cu) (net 18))
 (segment (start 15.355011 34.194988) (end 27.530022 34.194988) (width 0.25) (layer B.Cu) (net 18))
 (segment (start 30 36) (end 30 35.5) (width 0.25) (layer F.Cu) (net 18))
 (segment (start 30 35.5) (end 28.5 34) (width 0.25) (layer F.Cu) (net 18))
 (via (at 28.394693 33.919998) (size 0.8) (drill 0.4) (layers F.Cu B.Cu) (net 18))
 (segment (start 28.419998 33.919998) (end 28.394693 33.919998) (width 0.25) (layer F.Cu) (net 18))
 (segment (start 28.5 34) (end 28.419998 33.919998) (width 0.25) (layer F.Cu) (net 18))
 (segment (start 29 26.089999) (end 27.5 24.589999) (width 0.25) (layer B.Cu) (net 18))
 (segment (start 29 33.314691) (end 29 26.089999) (width 0.25) (layer B.Cu) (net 18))
 (segment (start 28.394693 33.919998) (end 29 33.314691) (width 0.25) (layer B.Cu) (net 18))
 (segment (start 27.805012 33.919998) (end 27.530022 34.194988) (width 0.25) (layer B.Cu) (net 18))
 (segment (start 28.394693 33.919998) (end 27.805012 33.919998) (width 0.25) (layer B.Cu) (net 18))
 (segment (start 45.546411 24.589999) (end 27.5 24.589999) (width 0.25) (layer F.Cu) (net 18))
 (segment (start 48.23 21.90641) (end 45.546411 24.589999) (width 0.25) (layer F.Cu) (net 18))
 (segment (start 48.23 11.5) (end 48.23 21.90641) (width 0.25) (layer F.Cu) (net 18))
 (via (at 28 12.5) (size 0.8) (drill 0.4) (layers F.Cu B.Cu) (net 33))
 (segment (start 28 14) (end 28 12.5) (width 0.25) (layer B.Cu) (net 33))
 (segment (start 28 12.5) (end 28 5) (width 0.25) (layer F.Cu) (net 33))
 (segment (start 25.46 9.0225) (end 25.5 9.0625) (width 0.25) (layer B.Cu) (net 34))
 (segment (start 25.46 5) (end 25.46 9.0225) (width 0.25) (layer B.Cu) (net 34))
 (segment (start 19.46 9.0225) (end 19.5 9.0625) (width 0.25) (layer B.Cu) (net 31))
 (segment (start 19.46 5) (end 19.46 9.0225) (width 0.25) (layer B.Cu) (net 31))
 (via (at 22 12.5) (size 0.8) (drill 0.4) (layers F.Cu B.Cu) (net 32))
 (segment (start 22 14) (end 22 12.5) (width 0.25) (layer B.Cu) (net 32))
 (segment (start 22 12.5) (end 22 5) (width 0.25) (layer F.Cu) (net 32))
 (segment (start 13.46 9.0225) (end 13.5 9.0625) (width 0.25) (layer B.Cu) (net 29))
 (segment (start 13.46 5) (end 13.46 9.0225) (width 0.25) (layer B.Cu) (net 29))
 (via (at 16 12.5) (size 0.8) (drill 0.4) (layers F.Cu B.Cu) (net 30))
 (segment (start 16 14) (end 16 12.5) (width 0.25) (layer B.Cu) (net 30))
 (segment (start 16 12.5) (end 16 5) (width 0.25) (layer F.Cu) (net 30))
 (segment (start 5.745001 20.527819) (end 5.745001 54.204999) (width 0.25) (layer B.Cu) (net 28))
 (segment (start 7.27282 19) (end 5.745001 20.527819) (width 0.25) (layer B.Cu) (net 28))
 (segment (start 5.745001 54.204999) (end 4.57 55.38) (width 0.25) (layer B.Cu) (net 28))
 (segment (start 22.5 19) (end 7.27282 19) (width 0.25) (layer B.Cu) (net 28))
 (segment (start 23.5 18) (end 22.5 19) (width 0.25) (layer B.Cu) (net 28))
 (segment (start 27.65 18) (end 23.5 18) (width 0.25) (layer B.Cu) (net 28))
 (segment (start 28.95 16.7) (end 27.65 18) (width 0.25) (layer B.Cu) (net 28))
 (segment (start 28.95 16) (end 28.95 16.7) (width 0.25) (layer B.Cu) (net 28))
 (segment (start 22 18.5) (end 22.95 17.55) (width 0.25) (layer B.Cu) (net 27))
 (segment (start 5.294991 20.341419) (end 7.13641 18.5) (width 0.25) (layer B.Cu) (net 27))
 (segment (start 5.294991 42.705009) (end 5.294991 20.341419) (width 0.25) (layer B.Cu) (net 27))
 (segment (start 3.394999 44.605001) (end 5.294991 42.705009) (width 0.25) (layer B.Cu) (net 27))
 (segment (start 7.13641 18.5) (end 22 18.5) (width 0.25) (layer B.Cu) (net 27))
 (segment (start 3.394999 51.664999) (end 3.394999 44.605001) (width 0.25) (layer B.Cu) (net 27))
 (segment (start 22.95 17.55) (end 22.95 16) (width 0.25) (layer B.Cu) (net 27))
 (segment (start 4.57 52.84) (end 3.394999 51.664999) (width 0.25) (layer B.Cu) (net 27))
 (segment (start 16.95 16) (end 16.95 17.05) (width 0.25) (layer B.Cu) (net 26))
 (segment (start 16.95 17.05) (end 16 18) (width 0.25) (layer B.Cu) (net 26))
 (segment (start 3.394999 49.124999) (end 3.394999 44.605001) (width 0.25) (layer F.Cu) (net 26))
 (segment (start 4.57 50.3) (end 3.394999 49.124999) (width 0.25) (layer F.Cu) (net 26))
 (via (at 4.5 42) (size 0.8) (drill 0.4) (layers F.Cu B.Cu) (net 26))
 (segment (start 4.5 43.5) (end 4.5 42) (width 0.25) (layer F.Cu) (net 26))
 (segment (start 3.394999 44.605001) (end 4.5 43.5) (width 0.25) (layer F.Cu) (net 26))
 (segment (start 4.5 41.344981) (end 4.5 42) (width 0.25) (layer B.Cu) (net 26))
 (segment (start 4.844981 41) (end 4.5 41.344981) (width 0.25) (layer B.Cu) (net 26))
 (segment (start 4.844981 23.60859) (end 4.844981 41) (width 0.25) (layer B.Cu) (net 26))
 (segment (start 4.844981 23.60859) (end 4.844981 20.155019) (width 0.25) (layer B.Cu) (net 26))
 (segment (start 4.844981 20.155019) (end 7 18) (width 0.25) (layer B.Cu) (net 26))
 (segment (start 7 18) (end 16 18) (width 0.25) (layer B.Cu) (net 26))
 (segment (start 39 3.5) (end 32.5 3.5) (width 0.25) (layer B.Cu) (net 23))
 (segment (start 36.5 6) (end 39 3.5) (width 0.25) (layer B.Cu) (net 23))
 (segment (start 36.5 53.5) (end 36.5 6) (width 0.25) (layer B.Cu) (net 23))
 (segment (start 35 55) (end 36.5 53.5) (width 0.25) (layer B.Cu) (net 23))
 (segment (start 28.5 55) (end 35 55) (width 0.25) (layer B.Cu) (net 23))
 (segment (start 28.12 55.38) (end 28.5 55) (width 0.25) (layer B.Cu) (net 23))
 (segment (start 27.43 55.38) (end 28.12 55.38) (width 0.25) (layer B.Cu) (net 23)))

